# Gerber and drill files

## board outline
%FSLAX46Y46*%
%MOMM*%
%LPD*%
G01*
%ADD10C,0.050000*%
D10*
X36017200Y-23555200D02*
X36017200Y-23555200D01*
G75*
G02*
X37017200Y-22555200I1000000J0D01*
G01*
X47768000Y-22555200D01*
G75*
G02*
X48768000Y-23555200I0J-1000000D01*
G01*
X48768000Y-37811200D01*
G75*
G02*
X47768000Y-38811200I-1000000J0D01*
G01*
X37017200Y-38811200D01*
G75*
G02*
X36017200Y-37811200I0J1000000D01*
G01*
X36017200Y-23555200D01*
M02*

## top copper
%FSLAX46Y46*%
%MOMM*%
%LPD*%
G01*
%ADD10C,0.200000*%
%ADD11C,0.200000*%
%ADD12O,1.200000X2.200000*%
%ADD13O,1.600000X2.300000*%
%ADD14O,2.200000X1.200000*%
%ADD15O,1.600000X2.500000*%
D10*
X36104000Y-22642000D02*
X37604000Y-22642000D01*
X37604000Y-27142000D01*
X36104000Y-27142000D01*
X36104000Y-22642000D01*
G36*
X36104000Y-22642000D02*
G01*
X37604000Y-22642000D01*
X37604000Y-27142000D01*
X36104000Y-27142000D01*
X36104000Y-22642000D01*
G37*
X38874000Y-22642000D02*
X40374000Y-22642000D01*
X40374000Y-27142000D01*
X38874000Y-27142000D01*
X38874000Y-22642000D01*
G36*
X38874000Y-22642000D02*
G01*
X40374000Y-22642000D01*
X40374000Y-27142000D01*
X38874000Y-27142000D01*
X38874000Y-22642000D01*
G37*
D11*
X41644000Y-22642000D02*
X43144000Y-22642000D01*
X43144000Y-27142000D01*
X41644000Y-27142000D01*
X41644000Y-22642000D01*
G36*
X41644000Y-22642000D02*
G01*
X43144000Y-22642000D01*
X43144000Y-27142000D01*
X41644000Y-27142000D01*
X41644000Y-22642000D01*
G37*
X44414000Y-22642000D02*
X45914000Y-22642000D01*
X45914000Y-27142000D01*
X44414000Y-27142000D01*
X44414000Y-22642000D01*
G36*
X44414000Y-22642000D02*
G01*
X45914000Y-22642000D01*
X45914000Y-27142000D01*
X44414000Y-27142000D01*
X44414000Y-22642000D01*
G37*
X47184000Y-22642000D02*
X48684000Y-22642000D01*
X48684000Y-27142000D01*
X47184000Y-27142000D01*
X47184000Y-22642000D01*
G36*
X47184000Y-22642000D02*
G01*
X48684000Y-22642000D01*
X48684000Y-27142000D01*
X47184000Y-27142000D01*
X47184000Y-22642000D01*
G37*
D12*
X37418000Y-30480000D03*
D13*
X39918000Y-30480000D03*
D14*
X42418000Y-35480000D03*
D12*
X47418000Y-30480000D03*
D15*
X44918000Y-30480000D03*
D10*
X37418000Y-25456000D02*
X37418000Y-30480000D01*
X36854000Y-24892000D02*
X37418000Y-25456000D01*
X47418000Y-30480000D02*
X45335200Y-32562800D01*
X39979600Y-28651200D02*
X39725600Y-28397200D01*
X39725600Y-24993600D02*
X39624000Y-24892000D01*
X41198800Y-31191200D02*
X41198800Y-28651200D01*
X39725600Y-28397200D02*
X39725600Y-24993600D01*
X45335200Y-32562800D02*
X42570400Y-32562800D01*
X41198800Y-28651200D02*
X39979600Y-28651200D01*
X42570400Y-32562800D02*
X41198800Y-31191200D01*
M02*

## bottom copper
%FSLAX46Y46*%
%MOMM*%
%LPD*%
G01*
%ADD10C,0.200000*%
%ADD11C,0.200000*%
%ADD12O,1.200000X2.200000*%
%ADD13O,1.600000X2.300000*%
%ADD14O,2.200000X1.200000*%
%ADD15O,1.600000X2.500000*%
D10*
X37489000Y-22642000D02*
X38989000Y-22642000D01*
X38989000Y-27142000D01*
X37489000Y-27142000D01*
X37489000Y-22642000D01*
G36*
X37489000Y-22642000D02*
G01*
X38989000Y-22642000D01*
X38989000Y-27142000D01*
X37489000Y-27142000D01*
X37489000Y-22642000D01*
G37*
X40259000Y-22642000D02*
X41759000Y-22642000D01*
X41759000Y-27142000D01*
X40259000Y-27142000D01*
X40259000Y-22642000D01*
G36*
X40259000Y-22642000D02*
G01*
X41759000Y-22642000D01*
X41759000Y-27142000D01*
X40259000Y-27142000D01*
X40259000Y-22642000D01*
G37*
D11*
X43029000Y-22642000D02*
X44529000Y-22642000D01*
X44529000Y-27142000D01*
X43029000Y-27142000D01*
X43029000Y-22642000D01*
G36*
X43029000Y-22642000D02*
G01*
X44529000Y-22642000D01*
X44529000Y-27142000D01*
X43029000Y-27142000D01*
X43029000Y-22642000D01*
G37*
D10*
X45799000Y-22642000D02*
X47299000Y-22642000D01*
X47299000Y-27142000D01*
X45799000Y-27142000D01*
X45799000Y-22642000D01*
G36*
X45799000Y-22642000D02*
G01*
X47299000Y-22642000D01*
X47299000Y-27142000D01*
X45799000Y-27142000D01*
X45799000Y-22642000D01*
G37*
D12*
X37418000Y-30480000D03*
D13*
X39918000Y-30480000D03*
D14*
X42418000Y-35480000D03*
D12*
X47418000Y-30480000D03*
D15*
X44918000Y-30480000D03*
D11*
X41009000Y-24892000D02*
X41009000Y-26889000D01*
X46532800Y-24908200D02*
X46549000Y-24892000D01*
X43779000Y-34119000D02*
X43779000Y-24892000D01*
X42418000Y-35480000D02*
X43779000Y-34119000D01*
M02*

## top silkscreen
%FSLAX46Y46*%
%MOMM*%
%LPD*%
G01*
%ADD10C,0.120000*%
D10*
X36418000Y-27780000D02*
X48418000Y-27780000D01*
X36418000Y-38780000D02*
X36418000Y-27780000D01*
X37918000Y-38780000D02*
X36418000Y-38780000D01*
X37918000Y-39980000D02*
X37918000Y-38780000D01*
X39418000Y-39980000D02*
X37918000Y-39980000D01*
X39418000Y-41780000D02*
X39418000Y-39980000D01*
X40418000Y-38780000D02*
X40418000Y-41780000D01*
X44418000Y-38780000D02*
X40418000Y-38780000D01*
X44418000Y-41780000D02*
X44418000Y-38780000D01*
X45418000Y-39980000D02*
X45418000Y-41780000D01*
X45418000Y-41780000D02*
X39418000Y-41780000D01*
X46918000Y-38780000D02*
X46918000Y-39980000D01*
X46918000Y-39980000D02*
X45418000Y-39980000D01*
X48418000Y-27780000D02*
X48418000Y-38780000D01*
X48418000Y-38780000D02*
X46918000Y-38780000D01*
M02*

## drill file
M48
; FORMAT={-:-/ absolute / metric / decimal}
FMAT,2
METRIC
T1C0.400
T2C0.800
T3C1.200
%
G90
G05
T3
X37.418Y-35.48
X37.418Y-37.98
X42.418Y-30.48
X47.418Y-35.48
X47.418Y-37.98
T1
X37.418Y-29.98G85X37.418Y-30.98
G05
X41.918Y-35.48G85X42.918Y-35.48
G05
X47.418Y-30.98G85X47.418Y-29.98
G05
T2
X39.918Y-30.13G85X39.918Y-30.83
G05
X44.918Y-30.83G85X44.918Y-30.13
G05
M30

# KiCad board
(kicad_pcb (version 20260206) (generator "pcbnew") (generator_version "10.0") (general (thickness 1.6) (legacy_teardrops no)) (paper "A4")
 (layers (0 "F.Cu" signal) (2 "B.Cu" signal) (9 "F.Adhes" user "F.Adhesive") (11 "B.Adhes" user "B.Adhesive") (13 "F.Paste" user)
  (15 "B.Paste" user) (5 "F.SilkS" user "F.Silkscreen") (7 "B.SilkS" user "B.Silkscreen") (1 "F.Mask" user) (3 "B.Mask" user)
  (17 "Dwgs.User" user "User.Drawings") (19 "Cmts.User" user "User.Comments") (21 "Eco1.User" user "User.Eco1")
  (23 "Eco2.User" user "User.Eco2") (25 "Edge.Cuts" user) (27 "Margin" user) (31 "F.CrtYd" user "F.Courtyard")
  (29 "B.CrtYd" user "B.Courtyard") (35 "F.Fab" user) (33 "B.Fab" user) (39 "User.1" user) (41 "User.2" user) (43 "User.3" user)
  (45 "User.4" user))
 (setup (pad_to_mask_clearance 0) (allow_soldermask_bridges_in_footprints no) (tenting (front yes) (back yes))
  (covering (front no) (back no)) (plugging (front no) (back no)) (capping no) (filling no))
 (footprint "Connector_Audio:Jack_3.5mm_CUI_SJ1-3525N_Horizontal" (layer "F.Cu") (at 42.418 35.48)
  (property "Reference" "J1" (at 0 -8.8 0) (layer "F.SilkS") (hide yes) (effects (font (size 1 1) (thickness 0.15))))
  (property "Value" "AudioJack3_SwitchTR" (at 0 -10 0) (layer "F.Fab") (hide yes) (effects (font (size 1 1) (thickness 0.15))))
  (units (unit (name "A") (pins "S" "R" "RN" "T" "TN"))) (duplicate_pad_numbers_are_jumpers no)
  (fp_line (start -6 -7.7) (end 6 -7.7) (stroke (width 0.12) (type solid)) (layer "F.SilkS"))
  (fp_line (start -6 3.3) (end -6 -7.7) (stroke (width 0.12) (type solid)) (layer "F.SilkS"))
  (fp_line (start -4.5 3.3) (end -6 3.3) (stroke (width 0.12) (type solid)) (layer "F.SilkS"))
  (fp_line (start -4.5 4.5) (end -4.5 3.3) (stroke (width 0.12) (type solid)) (layer "F.SilkS"))
  (fp_line (start -3 4.5) (end -4.5 4.5) (stroke (width 0.12) (type solid)) (layer "F.SilkS"))
  (fp_line (start -3 6.3) (end -3 4.5) (stroke (width 0.12) (type solid)) (layer "F.SilkS"))
  (fp_line (start -2 3.3) (end -2 6.3) (stroke (width 0.12) (type solid)) (layer "F.SilkS"))
  (fp_line (start 2 3.3) (end -2 3.3) (stroke (width 0.12) (type solid)) (layer "F.SilkS"))
  (fp_line (start 2 6.3) (end 2 3.3) (stroke (width 0.12) (type solid)) (layer "F.SilkS"))
  (fp_line (start 3 4.5) (end 3 6.3) (stroke (width 0.12) (type solid)) (layer "F.SilkS"))
  (fp_line (start 3 6.3) (end -3 6.3) (stroke (width 0.12) (type solid)) (layer "F.SilkS"))
  (fp_line (start 4.5 3.3) (end 4.5 4.5) (stroke (width 0.12) (type solid)) (layer "F.SilkS"))
  (fp_line (start 4.5 4.5) (end 3 4.5) (stroke (width 0.12) (type solid)) (layer "F.SilkS"))
  (fp_line (start 6 -7.7) (end 6 3.3) (stroke (width 0.12) (type solid)) (layer "F.SilkS"))
  (fp_line (start 6 3.3) (end 4.5 3.3) (stroke (width 0.12) (type solid)) (layer "F.SilkS"))
  (pad "" np_thru_hole circle (at -5 0) (size 1.2 1.2) (drill 1.2) (layers "*.Cu" "*.Mask"))
  (pad "" np_thru_hole circle (at -5 2.5) (size 1.2 1.2) (drill 1.2) (layers "*.Cu" "*.Mask"))
  (pad "" np_thru_hole circle (at 0 -5) (size 1.2 1.2) (drill 1.2) (layers "*.Cu" "*.Mask"))
  (pad "" np_thru_hole circle (at 5 0) (size 1.2 1.2) (drill 1.2) (layers "*.Cu" "*.Mask"))
  (pad "" np_thru_hole circle (at 5 2.5) (size 1.2 1.2) (drill 1.2) (layers "*.Cu" "*.Mask"))
  (pad "R" thru_hole oval (at -5 -5) (size 1.2 2.2) (drill oval 0.4 1.4) (layers "*.Cu" "*.Mask") (remove_unused_layers no) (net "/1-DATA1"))
  (pad "RN" thru_hole oval (at -2.5 -5) (size 1.6 2.3) (drill oval 0.8 1.5) (layers "*.Cu" "*.Mask") (remove_unused_layers no)
   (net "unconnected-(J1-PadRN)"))
  (pad "S" thru_hole oval (at 0 0) (size 2.2 1.2) (drill oval 1.4 0.4) (layers "*.Cu" "*.Mask") (remove_unused_layers no) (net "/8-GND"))
  (pad "T" thru_hole oval (at 5 -5 180) (size 1.2 2.2) (drill oval 0.4 1.4) (layers "*.Cu" "*.Mask") (remove_unused_layers no)
   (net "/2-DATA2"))
  (pad "TN" thru_hole oval (at 2.5 -5 180) (size 1.6 2.5) (drill oval 0.8 1.5) (layers "*.Cu" "*.Mask") (remove_unused_layers no)
   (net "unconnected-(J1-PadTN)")))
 (gr_rect (start 36.104 22.642) (end 37.604 27.142) (stroke (width 0.2) (type solid)) (fill yes) (layer "F.Cu") (net "/1-DATA1"))
 (gr_rect (start 38.874 22.642) (end 40.374 27.142) (stroke (width 0.2) (type solid)) (fill yes) (layer "F.Cu") (net "/2-DATA2"))
 (gr_rect (start 41.644 22.642) (end 43.144 27.142) (stroke (width 0.2) (type solid)) (fill yes) (layer "F.Cu"))
 (gr_rect (start 44.414 22.642) (end 45.914 27.142) (stroke (width 0.2) (type solid)) (fill yes) (layer "F.Cu"))
 (gr_rect (start 47.184 22.642) (end 48.684 27.142) (stroke (width 0.2) (type solid)) (fill yes) (layer "F.Cu"))
 (gr_rect (start 37.489 22.642) (end 38.989 27.142) (stroke (width 0.2) (type solid)) (fill yes) (layer "B.Cu"))
 (gr_rect (start 40.259 22.642) (end 41.759 27.142) (stroke (width 0.2) (type solid)) (fill yes) (layer "B.Cu"))
 (gr_rect (start 43.029 22.642) (end 44.529 27.142) (stroke (width 0.2) (type solid)) (fill yes) (layer "B.Cu") (net "/8-GND"))
 (gr_rect (start 45.799 22.642) (end 47.299 27.142) (stroke (width 0.2) (type solid)) (fill yes) (layer "B.Cu"))
 (gr_rect (start 36.0172 22.5552) (end 48.768 38.8112) (radius 1) (stroke (width 0.05) (type solid)) (fill no) (layer "Edge.Cuts"))
 (segment (start 41.009 24.892) (end 41.009 26.889) (width 0.2) (layer "B.Cu") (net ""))
 (segment (start 46.5328 24.9082) (end 46.549 24.892) (width 0.2) (layer "B.Cu") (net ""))
 (segment (start 37.418 25.456) (end 37.418 30.48) (width 0.2) (layer "F.Cu") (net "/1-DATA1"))
 (segment (start 36.854 24.892) (end 37.418 25.456) (width 0.2) (layer "F.Cu") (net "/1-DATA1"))
 (segment (start 43.779 34.119) (end 43.779 24.892) (width 0.2) (layer "B.Cu") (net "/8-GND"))
 (segment (start 42.418 35.48) (end 43.779 34.119) (width 0.2) (layer "B.Cu") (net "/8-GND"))
 (segment (start 47.418 30.48) (end 45.3352 32.5628) (width 0.2) (layer "F.Cu") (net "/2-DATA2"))
 (segment (start 39.9796 28.6512) (end 39.7256 28.3972) (width 0.2) (layer "F.Cu") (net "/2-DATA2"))
 (segment (start 39.7256 24.9936) (end 39.624 24.892) (width 0.2) (layer "F.Cu") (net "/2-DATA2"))
 (segment (start 41.1988 31.1912) (end 41.1988 28.6512) (width 0.2) (layer "F.Cu") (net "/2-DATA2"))
 (segment (start 39.7256 28.3972) (end 39.7256 24.9936) (width 0.2) (layer "F.Cu") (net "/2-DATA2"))
 (segment (start 45.3352 32.5628) (end 42.5704 32.5628) (width 0.2) (layer "F.Cu") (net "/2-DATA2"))
 (segment (start 41.1988 28.6512) (end 39.9796 28.6512) (width 0.2) (layer "F.Cu") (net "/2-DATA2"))
 (segment (start 42.5704 32.5628) (end 41.1988 31.1912) (width 0.2) (layer "F.Cu") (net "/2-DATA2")))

